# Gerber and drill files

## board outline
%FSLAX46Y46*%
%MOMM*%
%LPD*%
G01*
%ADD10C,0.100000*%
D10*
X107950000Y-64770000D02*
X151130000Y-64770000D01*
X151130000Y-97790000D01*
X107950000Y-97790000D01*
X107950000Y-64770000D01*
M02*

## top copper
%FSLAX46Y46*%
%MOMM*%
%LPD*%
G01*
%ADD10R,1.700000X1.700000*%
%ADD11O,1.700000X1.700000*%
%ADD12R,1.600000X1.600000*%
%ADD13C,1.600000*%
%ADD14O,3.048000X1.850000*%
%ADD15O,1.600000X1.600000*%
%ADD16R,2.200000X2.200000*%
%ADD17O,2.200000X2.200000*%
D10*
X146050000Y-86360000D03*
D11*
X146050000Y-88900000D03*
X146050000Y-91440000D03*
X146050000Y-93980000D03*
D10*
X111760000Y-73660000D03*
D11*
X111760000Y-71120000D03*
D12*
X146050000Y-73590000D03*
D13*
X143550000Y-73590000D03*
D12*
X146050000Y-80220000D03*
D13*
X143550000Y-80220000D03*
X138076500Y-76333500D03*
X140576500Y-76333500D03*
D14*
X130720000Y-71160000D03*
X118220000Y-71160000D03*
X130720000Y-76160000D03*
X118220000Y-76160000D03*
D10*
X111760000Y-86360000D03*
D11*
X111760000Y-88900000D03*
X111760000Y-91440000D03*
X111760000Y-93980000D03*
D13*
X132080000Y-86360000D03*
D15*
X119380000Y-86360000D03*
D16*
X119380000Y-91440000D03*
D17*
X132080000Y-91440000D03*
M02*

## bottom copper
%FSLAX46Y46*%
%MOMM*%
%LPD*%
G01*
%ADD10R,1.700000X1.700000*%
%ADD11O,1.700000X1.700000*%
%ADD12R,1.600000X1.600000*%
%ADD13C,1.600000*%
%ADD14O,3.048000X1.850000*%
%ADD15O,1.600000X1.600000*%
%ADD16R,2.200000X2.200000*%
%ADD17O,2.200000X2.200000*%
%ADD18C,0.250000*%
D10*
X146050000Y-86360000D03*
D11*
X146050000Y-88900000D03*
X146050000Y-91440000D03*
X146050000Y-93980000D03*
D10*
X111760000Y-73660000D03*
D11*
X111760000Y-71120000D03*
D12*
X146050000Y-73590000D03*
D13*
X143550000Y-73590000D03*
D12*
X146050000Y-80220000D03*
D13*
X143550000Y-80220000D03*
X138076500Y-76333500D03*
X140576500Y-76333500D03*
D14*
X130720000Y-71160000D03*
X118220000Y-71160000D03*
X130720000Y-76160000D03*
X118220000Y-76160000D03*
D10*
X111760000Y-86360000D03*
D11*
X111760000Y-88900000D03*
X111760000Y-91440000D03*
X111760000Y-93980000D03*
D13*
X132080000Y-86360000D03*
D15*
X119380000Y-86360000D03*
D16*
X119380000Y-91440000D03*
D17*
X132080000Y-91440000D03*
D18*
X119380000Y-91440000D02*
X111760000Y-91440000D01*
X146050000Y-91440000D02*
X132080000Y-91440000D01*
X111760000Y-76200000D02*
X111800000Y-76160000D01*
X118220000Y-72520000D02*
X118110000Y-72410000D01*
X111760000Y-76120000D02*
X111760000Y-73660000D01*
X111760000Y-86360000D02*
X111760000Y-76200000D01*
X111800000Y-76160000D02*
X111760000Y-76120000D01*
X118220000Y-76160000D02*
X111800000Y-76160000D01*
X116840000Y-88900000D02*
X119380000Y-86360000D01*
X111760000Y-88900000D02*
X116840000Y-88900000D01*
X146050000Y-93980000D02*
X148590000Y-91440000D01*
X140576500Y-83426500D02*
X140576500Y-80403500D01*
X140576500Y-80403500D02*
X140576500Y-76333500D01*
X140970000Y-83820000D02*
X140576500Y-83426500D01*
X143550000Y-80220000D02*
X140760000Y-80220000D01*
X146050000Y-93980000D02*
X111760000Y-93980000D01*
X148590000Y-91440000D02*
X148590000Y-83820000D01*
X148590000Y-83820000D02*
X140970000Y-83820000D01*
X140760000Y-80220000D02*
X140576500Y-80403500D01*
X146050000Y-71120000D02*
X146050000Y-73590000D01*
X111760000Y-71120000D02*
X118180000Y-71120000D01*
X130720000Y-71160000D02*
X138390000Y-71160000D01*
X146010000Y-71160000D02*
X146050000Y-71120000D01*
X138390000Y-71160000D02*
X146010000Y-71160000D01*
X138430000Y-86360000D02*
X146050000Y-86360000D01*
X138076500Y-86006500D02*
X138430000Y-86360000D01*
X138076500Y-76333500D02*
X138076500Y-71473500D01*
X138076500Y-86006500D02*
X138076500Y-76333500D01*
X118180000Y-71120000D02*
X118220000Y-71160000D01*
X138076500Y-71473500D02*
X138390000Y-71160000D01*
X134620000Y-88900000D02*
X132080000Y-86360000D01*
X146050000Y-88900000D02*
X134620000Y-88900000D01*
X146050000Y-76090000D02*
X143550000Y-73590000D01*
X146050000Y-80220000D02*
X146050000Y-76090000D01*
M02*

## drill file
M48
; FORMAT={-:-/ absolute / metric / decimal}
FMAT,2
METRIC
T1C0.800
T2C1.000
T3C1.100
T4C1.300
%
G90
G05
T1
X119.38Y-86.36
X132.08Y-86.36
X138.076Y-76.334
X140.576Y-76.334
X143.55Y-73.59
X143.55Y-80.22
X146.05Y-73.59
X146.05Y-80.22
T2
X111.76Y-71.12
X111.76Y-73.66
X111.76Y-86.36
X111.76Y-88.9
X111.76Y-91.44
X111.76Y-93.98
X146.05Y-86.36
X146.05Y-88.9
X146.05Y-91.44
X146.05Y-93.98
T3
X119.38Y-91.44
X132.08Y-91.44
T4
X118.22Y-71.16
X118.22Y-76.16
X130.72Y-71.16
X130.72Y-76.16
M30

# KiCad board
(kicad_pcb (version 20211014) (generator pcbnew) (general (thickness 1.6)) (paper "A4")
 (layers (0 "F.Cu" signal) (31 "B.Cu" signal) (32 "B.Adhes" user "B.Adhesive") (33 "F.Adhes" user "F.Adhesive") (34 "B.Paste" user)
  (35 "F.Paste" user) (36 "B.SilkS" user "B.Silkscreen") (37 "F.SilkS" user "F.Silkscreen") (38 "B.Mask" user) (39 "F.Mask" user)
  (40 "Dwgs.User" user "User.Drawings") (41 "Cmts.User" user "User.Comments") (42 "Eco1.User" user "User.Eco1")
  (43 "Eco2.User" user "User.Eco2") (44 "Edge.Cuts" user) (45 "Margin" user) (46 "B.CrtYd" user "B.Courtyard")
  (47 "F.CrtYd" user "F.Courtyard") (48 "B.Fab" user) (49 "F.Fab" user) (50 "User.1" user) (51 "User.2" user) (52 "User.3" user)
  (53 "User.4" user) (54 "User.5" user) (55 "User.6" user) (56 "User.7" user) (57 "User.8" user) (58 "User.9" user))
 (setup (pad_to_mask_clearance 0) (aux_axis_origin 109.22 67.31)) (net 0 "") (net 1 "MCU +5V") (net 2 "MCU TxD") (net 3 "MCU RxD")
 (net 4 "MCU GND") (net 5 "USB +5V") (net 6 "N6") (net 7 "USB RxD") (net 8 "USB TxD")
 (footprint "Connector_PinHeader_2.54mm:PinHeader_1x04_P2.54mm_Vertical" (layer "F.Cu") (at 146.05 86.36)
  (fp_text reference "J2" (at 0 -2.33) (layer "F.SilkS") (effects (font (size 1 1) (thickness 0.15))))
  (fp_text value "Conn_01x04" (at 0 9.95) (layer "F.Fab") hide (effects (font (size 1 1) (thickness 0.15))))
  (pad "1" thru_hole rect (at 0 0) (size 1.7 1.7) (drill 1) (layers *.Cu *.Mask) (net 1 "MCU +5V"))
  (pad "2" thru_hole oval (at 0 2.54) (size 1.7 1.7) (drill 1) (layers *.Cu *.Mask) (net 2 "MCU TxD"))
  (pad "3" thru_hole oval (at 0 5.08) (size 1.7 1.7) (drill 1) (layers *.Cu *.Mask) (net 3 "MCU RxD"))
  (pad "4" thru_hole oval (at 0 7.62) (size 1.7 1.7) (drill 1) (layers *.Cu *.Mask) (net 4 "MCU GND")))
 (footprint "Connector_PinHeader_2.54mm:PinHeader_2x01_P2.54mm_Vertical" (layer "F.Cu") (at 111.76 73.66 90)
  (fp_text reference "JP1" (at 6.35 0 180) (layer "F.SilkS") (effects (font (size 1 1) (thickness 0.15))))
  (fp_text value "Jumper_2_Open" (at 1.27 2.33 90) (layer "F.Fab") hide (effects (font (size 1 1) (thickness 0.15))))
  (pad "1" thru_hole rect (at 0 0 90) (size 1.7 1.7) (drill 1) (layers *.Cu *.Mask) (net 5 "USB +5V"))
  (pad "2" thru_hole oval (at 2.54 0 90) (size 1.7 1.7) (drill 1) (layers *.Cu *.Mask) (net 1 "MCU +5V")))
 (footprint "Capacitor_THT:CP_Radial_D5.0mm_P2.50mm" (layer "F.Cu") (at 146.05 73.59 180)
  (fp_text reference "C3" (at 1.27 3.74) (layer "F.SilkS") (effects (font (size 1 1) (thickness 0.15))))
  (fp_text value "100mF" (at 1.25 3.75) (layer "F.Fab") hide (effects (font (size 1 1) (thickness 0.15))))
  (pad "1" thru_hole rect (at 0 0 180) (size 1.6 1.6) (drill 0.8) (layers *.Cu *.Mask) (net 1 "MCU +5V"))
  (pad "2" thru_hole circle (at 2.5 0 180) (size 1.6 1.6) (drill 0.8) (layers *.Cu *.Mask) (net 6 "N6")))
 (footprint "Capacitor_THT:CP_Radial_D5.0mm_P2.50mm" (layer "F.Cu") (at 146.05 80.22 180)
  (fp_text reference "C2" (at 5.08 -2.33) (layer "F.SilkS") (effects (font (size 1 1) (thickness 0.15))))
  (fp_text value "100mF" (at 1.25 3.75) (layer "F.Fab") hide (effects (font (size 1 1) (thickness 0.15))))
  (pad "1" thru_hole rect (at 0 0 180) (size 1.6 1.6) (drill 0.8) (layers *.Cu *.Mask) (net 6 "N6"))
  (pad "2" thru_hole circle (at 2.5 0 180) (size 1.6 1.6) (drill 0.8) (layers *.Cu *.Mask) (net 4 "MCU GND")))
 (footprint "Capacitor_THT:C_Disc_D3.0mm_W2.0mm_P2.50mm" (layer "F.Cu") (at 138.0765 76.3335)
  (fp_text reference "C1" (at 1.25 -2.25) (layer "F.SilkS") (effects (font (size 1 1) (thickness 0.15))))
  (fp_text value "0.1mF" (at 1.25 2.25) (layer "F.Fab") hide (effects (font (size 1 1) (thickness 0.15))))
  (pad "1" thru_hole circle (at 0 0) (size 1.6 1.6) (drill 0.8) (layers *.Cu *.Mask) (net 1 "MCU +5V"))
  (pad "2" thru_hole circle (at 2.5 0) (size 1.6 1.6) (drill 0.8) (layers *.Cu *.Mask) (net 4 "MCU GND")))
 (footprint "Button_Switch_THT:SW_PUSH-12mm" (layer "F.Cu") (at 118.22 71.16)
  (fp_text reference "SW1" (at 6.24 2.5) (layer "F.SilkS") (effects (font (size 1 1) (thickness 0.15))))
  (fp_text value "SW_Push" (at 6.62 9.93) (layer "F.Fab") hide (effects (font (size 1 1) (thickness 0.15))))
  (pad "1" thru_hole oval (at 12.5 0) (size 3.048 1.85) (drill 1.3) (layers *.Cu *.Mask) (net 1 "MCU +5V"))
  (pad "1" thru_hole oval (at 0 0) (size 3.048 1.85) (drill 1.3) (layers *.Cu *.Mask) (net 1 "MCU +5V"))
  (pad "2" thru_hole oval (at 12.5 5) (size 3.048 1.85) (drill 1.3) (layers *.Cu *.Mask) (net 5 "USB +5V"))
  (pad "2" thru_hole oval (at 0 5) (size 3.048 1.85) (drill 1.3) (layers *.Cu *.Mask) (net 5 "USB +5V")))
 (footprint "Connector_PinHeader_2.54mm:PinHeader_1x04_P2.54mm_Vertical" (layer "F.Cu") (at 111.76 86.36)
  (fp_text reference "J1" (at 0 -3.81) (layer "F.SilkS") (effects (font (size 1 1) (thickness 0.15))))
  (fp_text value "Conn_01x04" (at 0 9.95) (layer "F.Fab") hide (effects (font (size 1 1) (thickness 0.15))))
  (pad "1" thru_hole rect (at 0 0) (size 1.7 1.7) (drill 1) (layers *.Cu *.Mask) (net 5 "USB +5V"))
  (pad "2" thru_hole oval (at 0 2.54) (size 1.7 1.7) (drill 1) (layers *.Cu *.Mask) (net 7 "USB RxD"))
  (pad "3" thru_hole oval (at 0 5.08) (size 1.7 1.7) (drill 1) (layers *.Cu *.Mask) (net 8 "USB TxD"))
  (pad "4" thru_hole oval (at 0 7.62) (size 1.7 1.7) (drill 1) (layers *.Cu *.Mask) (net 4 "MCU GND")))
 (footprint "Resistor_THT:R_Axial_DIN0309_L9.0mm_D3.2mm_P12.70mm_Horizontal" (layer "F.Cu") (at 132.08 86.36 180)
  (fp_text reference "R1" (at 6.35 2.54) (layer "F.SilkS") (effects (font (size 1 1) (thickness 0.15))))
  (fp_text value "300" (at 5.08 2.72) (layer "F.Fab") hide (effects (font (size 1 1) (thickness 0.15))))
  (pad "1" thru_hole circle (at 0 0 180) (size 1.6 1.6) (drill 0.8) (layers *.Cu *.Mask) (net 2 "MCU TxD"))
  (pad "2" thru_hole oval (at 12.7 0 180) (size 1.6 1.6) (drill 0.8) (layers *.Cu *.Mask) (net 7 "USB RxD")))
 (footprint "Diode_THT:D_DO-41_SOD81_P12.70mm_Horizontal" (layer "F.Cu") (at 119.38 91.44)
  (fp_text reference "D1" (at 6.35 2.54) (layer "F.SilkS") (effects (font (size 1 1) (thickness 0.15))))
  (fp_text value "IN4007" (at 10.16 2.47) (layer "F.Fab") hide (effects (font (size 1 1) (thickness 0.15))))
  (pad "1" thru_hole rect (at 0 0) (size 2.2 2.2) (drill 1.1) (layers *.Cu *.Mask) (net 8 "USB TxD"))
  (pad "2" thru_hole oval (at 12.7 0) (size 2.2 2.2) (drill 1.1) (layers *.Cu *.Mask) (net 3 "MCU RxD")))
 (gr_rect (start 107.95 64.77) (end 151.13 97.79) (layer "Edge.Cuts") (width 0.1) (fill none))
 (segment (start 119.38 91.44) (end 111.76 91.44) (width 0.25) (layer "B.Cu") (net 8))
 (segment (start 146.05 91.44) (end 132.08 91.44) (width 0.25) (layer "B.Cu") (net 3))
 (segment (start 111.76 76.2) (end 111.8 76.16) (width 0.25) (layer "B.Cu") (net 5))
 (segment (start 118.22 72.52) (end 118.11 72.41) (width 0.25) (layer "B.Cu") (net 5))
 (segment (start 111.76 76.12) (end 111.76 73.66) (width 0.25) (layer "B.Cu") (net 5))
 (segment (start 111.76 86.36) (end 111.76 76.2) (width 0.25) (layer "B.Cu") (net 5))
 (segment (start 111.8 76.16) (end 111.76 76.12) (width 0.25) (layer "B.Cu") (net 5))
 (segment (start 118.22 76.16) (end 111.8 76.16) (width 0.25) (layer "B.Cu") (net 5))
 (segment (start 116.84 88.9) (end 119.38 86.36) (width 0.25) (layer "B.Cu") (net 7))
 (segment (start 111.76 88.9) (end 116.84 88.9) (width 0.25) (layer "B.Cu") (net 7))
 (segment (start 146.05 93.98) (end 148.59 91.44) (width 0.25) (layer "B.Cu") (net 4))
 (segment (start 140.5765 83.4265) (end 140.5765 80.4035) (width 0.25) (layer "B.Cu") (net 4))
 (segment (start 140.5765 80.4035) (end 140.5765 76.3335) (width 0.25) (layer "B.Cu") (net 4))
 (segment (start 140.97 83.82) (end 140.5765 83.4265) (width 0.25) (layer "B.Cu") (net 4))
 (segment (start 143.55 80.22) (end 140.76 80.22) (width 0.25) (layer "B.Cu") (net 4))
 (segment (start 146.05 93.98) (end 111.76 93.98) (width 0.25) (layer "B.Cu") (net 4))
 (segment (start 148.59 91.44) (end 148.59 83.82) (width 0.25) (layer "B.Cu") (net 4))
 (segment (start 148.59 83.82) (end 140.97 83.82) (width 0.25) (layer "B.Cu") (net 4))
 (segment (start 140.76 80.22) (end 140.5765 80.4035) (width 0.25) (layer "B.Cu") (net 4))
 (segment (start 146.05 71.12) (end 146.05 73.59) (width 0.25) (layer "B.Cu") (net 1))
 (segment (start 111.76 71.12) (end 118.18 71.12) (width 0.25) (layer "B.Cu") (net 1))
 (segment (start 130.72 71.16) (end 138.39 71.16) (width 0.25) (layer "B.Cu") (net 1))
 (segment (start 146.01 71.16) (end 146.05 71.12) (width 0.25) (layer "B.Cu") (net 1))
 (segment (start 138.39 71.16) (end 146.01 71.16) (width 0.25) (layer "B.Cu") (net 1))
 (segment (start 138.43 86.36) (end 146.05 86.36) (width 0.25) (layer "B.Cu") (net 1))
 (segment (start 138.0765 86.0065) (end 138.43 86.36) (width 0.25) (layer "B.Cu") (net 1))
 (segment (start 138.0765 76.3335) (end 138.0765 71.4735) (width 0.25) (layer "B.Cu") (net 1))
 (segment (start 138.0765 86.0065) (end 138.0765 76.3335) (width 0.25) (layer "B.Cu") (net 1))
 (segment (start 118.18 71.12) (end 118.22 71.16) (width 0.25) (layer "B.Cu") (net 1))
 (segment (start 138.0765 71.4735) (end 138.39 71.16) (width 0.25) (layer "B.Cu") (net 1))
 (segment (start 134.62 88.9) (end 132.08 86.36) (width 0.25) (layer "B.Cu") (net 2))
 (segment (start 146.05 88.9) (end 134.62 88.9) (width 0.25) (layer "B.Cu") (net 2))
 (segment (start 146.05 76.09) (end 143.55 73.59) (width 0.25) (layer "B.Cu") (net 6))
 (segment (start 146.05 80.22) (end 146.05 76.09) (width 0.25) (layer "B.Cu") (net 6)))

